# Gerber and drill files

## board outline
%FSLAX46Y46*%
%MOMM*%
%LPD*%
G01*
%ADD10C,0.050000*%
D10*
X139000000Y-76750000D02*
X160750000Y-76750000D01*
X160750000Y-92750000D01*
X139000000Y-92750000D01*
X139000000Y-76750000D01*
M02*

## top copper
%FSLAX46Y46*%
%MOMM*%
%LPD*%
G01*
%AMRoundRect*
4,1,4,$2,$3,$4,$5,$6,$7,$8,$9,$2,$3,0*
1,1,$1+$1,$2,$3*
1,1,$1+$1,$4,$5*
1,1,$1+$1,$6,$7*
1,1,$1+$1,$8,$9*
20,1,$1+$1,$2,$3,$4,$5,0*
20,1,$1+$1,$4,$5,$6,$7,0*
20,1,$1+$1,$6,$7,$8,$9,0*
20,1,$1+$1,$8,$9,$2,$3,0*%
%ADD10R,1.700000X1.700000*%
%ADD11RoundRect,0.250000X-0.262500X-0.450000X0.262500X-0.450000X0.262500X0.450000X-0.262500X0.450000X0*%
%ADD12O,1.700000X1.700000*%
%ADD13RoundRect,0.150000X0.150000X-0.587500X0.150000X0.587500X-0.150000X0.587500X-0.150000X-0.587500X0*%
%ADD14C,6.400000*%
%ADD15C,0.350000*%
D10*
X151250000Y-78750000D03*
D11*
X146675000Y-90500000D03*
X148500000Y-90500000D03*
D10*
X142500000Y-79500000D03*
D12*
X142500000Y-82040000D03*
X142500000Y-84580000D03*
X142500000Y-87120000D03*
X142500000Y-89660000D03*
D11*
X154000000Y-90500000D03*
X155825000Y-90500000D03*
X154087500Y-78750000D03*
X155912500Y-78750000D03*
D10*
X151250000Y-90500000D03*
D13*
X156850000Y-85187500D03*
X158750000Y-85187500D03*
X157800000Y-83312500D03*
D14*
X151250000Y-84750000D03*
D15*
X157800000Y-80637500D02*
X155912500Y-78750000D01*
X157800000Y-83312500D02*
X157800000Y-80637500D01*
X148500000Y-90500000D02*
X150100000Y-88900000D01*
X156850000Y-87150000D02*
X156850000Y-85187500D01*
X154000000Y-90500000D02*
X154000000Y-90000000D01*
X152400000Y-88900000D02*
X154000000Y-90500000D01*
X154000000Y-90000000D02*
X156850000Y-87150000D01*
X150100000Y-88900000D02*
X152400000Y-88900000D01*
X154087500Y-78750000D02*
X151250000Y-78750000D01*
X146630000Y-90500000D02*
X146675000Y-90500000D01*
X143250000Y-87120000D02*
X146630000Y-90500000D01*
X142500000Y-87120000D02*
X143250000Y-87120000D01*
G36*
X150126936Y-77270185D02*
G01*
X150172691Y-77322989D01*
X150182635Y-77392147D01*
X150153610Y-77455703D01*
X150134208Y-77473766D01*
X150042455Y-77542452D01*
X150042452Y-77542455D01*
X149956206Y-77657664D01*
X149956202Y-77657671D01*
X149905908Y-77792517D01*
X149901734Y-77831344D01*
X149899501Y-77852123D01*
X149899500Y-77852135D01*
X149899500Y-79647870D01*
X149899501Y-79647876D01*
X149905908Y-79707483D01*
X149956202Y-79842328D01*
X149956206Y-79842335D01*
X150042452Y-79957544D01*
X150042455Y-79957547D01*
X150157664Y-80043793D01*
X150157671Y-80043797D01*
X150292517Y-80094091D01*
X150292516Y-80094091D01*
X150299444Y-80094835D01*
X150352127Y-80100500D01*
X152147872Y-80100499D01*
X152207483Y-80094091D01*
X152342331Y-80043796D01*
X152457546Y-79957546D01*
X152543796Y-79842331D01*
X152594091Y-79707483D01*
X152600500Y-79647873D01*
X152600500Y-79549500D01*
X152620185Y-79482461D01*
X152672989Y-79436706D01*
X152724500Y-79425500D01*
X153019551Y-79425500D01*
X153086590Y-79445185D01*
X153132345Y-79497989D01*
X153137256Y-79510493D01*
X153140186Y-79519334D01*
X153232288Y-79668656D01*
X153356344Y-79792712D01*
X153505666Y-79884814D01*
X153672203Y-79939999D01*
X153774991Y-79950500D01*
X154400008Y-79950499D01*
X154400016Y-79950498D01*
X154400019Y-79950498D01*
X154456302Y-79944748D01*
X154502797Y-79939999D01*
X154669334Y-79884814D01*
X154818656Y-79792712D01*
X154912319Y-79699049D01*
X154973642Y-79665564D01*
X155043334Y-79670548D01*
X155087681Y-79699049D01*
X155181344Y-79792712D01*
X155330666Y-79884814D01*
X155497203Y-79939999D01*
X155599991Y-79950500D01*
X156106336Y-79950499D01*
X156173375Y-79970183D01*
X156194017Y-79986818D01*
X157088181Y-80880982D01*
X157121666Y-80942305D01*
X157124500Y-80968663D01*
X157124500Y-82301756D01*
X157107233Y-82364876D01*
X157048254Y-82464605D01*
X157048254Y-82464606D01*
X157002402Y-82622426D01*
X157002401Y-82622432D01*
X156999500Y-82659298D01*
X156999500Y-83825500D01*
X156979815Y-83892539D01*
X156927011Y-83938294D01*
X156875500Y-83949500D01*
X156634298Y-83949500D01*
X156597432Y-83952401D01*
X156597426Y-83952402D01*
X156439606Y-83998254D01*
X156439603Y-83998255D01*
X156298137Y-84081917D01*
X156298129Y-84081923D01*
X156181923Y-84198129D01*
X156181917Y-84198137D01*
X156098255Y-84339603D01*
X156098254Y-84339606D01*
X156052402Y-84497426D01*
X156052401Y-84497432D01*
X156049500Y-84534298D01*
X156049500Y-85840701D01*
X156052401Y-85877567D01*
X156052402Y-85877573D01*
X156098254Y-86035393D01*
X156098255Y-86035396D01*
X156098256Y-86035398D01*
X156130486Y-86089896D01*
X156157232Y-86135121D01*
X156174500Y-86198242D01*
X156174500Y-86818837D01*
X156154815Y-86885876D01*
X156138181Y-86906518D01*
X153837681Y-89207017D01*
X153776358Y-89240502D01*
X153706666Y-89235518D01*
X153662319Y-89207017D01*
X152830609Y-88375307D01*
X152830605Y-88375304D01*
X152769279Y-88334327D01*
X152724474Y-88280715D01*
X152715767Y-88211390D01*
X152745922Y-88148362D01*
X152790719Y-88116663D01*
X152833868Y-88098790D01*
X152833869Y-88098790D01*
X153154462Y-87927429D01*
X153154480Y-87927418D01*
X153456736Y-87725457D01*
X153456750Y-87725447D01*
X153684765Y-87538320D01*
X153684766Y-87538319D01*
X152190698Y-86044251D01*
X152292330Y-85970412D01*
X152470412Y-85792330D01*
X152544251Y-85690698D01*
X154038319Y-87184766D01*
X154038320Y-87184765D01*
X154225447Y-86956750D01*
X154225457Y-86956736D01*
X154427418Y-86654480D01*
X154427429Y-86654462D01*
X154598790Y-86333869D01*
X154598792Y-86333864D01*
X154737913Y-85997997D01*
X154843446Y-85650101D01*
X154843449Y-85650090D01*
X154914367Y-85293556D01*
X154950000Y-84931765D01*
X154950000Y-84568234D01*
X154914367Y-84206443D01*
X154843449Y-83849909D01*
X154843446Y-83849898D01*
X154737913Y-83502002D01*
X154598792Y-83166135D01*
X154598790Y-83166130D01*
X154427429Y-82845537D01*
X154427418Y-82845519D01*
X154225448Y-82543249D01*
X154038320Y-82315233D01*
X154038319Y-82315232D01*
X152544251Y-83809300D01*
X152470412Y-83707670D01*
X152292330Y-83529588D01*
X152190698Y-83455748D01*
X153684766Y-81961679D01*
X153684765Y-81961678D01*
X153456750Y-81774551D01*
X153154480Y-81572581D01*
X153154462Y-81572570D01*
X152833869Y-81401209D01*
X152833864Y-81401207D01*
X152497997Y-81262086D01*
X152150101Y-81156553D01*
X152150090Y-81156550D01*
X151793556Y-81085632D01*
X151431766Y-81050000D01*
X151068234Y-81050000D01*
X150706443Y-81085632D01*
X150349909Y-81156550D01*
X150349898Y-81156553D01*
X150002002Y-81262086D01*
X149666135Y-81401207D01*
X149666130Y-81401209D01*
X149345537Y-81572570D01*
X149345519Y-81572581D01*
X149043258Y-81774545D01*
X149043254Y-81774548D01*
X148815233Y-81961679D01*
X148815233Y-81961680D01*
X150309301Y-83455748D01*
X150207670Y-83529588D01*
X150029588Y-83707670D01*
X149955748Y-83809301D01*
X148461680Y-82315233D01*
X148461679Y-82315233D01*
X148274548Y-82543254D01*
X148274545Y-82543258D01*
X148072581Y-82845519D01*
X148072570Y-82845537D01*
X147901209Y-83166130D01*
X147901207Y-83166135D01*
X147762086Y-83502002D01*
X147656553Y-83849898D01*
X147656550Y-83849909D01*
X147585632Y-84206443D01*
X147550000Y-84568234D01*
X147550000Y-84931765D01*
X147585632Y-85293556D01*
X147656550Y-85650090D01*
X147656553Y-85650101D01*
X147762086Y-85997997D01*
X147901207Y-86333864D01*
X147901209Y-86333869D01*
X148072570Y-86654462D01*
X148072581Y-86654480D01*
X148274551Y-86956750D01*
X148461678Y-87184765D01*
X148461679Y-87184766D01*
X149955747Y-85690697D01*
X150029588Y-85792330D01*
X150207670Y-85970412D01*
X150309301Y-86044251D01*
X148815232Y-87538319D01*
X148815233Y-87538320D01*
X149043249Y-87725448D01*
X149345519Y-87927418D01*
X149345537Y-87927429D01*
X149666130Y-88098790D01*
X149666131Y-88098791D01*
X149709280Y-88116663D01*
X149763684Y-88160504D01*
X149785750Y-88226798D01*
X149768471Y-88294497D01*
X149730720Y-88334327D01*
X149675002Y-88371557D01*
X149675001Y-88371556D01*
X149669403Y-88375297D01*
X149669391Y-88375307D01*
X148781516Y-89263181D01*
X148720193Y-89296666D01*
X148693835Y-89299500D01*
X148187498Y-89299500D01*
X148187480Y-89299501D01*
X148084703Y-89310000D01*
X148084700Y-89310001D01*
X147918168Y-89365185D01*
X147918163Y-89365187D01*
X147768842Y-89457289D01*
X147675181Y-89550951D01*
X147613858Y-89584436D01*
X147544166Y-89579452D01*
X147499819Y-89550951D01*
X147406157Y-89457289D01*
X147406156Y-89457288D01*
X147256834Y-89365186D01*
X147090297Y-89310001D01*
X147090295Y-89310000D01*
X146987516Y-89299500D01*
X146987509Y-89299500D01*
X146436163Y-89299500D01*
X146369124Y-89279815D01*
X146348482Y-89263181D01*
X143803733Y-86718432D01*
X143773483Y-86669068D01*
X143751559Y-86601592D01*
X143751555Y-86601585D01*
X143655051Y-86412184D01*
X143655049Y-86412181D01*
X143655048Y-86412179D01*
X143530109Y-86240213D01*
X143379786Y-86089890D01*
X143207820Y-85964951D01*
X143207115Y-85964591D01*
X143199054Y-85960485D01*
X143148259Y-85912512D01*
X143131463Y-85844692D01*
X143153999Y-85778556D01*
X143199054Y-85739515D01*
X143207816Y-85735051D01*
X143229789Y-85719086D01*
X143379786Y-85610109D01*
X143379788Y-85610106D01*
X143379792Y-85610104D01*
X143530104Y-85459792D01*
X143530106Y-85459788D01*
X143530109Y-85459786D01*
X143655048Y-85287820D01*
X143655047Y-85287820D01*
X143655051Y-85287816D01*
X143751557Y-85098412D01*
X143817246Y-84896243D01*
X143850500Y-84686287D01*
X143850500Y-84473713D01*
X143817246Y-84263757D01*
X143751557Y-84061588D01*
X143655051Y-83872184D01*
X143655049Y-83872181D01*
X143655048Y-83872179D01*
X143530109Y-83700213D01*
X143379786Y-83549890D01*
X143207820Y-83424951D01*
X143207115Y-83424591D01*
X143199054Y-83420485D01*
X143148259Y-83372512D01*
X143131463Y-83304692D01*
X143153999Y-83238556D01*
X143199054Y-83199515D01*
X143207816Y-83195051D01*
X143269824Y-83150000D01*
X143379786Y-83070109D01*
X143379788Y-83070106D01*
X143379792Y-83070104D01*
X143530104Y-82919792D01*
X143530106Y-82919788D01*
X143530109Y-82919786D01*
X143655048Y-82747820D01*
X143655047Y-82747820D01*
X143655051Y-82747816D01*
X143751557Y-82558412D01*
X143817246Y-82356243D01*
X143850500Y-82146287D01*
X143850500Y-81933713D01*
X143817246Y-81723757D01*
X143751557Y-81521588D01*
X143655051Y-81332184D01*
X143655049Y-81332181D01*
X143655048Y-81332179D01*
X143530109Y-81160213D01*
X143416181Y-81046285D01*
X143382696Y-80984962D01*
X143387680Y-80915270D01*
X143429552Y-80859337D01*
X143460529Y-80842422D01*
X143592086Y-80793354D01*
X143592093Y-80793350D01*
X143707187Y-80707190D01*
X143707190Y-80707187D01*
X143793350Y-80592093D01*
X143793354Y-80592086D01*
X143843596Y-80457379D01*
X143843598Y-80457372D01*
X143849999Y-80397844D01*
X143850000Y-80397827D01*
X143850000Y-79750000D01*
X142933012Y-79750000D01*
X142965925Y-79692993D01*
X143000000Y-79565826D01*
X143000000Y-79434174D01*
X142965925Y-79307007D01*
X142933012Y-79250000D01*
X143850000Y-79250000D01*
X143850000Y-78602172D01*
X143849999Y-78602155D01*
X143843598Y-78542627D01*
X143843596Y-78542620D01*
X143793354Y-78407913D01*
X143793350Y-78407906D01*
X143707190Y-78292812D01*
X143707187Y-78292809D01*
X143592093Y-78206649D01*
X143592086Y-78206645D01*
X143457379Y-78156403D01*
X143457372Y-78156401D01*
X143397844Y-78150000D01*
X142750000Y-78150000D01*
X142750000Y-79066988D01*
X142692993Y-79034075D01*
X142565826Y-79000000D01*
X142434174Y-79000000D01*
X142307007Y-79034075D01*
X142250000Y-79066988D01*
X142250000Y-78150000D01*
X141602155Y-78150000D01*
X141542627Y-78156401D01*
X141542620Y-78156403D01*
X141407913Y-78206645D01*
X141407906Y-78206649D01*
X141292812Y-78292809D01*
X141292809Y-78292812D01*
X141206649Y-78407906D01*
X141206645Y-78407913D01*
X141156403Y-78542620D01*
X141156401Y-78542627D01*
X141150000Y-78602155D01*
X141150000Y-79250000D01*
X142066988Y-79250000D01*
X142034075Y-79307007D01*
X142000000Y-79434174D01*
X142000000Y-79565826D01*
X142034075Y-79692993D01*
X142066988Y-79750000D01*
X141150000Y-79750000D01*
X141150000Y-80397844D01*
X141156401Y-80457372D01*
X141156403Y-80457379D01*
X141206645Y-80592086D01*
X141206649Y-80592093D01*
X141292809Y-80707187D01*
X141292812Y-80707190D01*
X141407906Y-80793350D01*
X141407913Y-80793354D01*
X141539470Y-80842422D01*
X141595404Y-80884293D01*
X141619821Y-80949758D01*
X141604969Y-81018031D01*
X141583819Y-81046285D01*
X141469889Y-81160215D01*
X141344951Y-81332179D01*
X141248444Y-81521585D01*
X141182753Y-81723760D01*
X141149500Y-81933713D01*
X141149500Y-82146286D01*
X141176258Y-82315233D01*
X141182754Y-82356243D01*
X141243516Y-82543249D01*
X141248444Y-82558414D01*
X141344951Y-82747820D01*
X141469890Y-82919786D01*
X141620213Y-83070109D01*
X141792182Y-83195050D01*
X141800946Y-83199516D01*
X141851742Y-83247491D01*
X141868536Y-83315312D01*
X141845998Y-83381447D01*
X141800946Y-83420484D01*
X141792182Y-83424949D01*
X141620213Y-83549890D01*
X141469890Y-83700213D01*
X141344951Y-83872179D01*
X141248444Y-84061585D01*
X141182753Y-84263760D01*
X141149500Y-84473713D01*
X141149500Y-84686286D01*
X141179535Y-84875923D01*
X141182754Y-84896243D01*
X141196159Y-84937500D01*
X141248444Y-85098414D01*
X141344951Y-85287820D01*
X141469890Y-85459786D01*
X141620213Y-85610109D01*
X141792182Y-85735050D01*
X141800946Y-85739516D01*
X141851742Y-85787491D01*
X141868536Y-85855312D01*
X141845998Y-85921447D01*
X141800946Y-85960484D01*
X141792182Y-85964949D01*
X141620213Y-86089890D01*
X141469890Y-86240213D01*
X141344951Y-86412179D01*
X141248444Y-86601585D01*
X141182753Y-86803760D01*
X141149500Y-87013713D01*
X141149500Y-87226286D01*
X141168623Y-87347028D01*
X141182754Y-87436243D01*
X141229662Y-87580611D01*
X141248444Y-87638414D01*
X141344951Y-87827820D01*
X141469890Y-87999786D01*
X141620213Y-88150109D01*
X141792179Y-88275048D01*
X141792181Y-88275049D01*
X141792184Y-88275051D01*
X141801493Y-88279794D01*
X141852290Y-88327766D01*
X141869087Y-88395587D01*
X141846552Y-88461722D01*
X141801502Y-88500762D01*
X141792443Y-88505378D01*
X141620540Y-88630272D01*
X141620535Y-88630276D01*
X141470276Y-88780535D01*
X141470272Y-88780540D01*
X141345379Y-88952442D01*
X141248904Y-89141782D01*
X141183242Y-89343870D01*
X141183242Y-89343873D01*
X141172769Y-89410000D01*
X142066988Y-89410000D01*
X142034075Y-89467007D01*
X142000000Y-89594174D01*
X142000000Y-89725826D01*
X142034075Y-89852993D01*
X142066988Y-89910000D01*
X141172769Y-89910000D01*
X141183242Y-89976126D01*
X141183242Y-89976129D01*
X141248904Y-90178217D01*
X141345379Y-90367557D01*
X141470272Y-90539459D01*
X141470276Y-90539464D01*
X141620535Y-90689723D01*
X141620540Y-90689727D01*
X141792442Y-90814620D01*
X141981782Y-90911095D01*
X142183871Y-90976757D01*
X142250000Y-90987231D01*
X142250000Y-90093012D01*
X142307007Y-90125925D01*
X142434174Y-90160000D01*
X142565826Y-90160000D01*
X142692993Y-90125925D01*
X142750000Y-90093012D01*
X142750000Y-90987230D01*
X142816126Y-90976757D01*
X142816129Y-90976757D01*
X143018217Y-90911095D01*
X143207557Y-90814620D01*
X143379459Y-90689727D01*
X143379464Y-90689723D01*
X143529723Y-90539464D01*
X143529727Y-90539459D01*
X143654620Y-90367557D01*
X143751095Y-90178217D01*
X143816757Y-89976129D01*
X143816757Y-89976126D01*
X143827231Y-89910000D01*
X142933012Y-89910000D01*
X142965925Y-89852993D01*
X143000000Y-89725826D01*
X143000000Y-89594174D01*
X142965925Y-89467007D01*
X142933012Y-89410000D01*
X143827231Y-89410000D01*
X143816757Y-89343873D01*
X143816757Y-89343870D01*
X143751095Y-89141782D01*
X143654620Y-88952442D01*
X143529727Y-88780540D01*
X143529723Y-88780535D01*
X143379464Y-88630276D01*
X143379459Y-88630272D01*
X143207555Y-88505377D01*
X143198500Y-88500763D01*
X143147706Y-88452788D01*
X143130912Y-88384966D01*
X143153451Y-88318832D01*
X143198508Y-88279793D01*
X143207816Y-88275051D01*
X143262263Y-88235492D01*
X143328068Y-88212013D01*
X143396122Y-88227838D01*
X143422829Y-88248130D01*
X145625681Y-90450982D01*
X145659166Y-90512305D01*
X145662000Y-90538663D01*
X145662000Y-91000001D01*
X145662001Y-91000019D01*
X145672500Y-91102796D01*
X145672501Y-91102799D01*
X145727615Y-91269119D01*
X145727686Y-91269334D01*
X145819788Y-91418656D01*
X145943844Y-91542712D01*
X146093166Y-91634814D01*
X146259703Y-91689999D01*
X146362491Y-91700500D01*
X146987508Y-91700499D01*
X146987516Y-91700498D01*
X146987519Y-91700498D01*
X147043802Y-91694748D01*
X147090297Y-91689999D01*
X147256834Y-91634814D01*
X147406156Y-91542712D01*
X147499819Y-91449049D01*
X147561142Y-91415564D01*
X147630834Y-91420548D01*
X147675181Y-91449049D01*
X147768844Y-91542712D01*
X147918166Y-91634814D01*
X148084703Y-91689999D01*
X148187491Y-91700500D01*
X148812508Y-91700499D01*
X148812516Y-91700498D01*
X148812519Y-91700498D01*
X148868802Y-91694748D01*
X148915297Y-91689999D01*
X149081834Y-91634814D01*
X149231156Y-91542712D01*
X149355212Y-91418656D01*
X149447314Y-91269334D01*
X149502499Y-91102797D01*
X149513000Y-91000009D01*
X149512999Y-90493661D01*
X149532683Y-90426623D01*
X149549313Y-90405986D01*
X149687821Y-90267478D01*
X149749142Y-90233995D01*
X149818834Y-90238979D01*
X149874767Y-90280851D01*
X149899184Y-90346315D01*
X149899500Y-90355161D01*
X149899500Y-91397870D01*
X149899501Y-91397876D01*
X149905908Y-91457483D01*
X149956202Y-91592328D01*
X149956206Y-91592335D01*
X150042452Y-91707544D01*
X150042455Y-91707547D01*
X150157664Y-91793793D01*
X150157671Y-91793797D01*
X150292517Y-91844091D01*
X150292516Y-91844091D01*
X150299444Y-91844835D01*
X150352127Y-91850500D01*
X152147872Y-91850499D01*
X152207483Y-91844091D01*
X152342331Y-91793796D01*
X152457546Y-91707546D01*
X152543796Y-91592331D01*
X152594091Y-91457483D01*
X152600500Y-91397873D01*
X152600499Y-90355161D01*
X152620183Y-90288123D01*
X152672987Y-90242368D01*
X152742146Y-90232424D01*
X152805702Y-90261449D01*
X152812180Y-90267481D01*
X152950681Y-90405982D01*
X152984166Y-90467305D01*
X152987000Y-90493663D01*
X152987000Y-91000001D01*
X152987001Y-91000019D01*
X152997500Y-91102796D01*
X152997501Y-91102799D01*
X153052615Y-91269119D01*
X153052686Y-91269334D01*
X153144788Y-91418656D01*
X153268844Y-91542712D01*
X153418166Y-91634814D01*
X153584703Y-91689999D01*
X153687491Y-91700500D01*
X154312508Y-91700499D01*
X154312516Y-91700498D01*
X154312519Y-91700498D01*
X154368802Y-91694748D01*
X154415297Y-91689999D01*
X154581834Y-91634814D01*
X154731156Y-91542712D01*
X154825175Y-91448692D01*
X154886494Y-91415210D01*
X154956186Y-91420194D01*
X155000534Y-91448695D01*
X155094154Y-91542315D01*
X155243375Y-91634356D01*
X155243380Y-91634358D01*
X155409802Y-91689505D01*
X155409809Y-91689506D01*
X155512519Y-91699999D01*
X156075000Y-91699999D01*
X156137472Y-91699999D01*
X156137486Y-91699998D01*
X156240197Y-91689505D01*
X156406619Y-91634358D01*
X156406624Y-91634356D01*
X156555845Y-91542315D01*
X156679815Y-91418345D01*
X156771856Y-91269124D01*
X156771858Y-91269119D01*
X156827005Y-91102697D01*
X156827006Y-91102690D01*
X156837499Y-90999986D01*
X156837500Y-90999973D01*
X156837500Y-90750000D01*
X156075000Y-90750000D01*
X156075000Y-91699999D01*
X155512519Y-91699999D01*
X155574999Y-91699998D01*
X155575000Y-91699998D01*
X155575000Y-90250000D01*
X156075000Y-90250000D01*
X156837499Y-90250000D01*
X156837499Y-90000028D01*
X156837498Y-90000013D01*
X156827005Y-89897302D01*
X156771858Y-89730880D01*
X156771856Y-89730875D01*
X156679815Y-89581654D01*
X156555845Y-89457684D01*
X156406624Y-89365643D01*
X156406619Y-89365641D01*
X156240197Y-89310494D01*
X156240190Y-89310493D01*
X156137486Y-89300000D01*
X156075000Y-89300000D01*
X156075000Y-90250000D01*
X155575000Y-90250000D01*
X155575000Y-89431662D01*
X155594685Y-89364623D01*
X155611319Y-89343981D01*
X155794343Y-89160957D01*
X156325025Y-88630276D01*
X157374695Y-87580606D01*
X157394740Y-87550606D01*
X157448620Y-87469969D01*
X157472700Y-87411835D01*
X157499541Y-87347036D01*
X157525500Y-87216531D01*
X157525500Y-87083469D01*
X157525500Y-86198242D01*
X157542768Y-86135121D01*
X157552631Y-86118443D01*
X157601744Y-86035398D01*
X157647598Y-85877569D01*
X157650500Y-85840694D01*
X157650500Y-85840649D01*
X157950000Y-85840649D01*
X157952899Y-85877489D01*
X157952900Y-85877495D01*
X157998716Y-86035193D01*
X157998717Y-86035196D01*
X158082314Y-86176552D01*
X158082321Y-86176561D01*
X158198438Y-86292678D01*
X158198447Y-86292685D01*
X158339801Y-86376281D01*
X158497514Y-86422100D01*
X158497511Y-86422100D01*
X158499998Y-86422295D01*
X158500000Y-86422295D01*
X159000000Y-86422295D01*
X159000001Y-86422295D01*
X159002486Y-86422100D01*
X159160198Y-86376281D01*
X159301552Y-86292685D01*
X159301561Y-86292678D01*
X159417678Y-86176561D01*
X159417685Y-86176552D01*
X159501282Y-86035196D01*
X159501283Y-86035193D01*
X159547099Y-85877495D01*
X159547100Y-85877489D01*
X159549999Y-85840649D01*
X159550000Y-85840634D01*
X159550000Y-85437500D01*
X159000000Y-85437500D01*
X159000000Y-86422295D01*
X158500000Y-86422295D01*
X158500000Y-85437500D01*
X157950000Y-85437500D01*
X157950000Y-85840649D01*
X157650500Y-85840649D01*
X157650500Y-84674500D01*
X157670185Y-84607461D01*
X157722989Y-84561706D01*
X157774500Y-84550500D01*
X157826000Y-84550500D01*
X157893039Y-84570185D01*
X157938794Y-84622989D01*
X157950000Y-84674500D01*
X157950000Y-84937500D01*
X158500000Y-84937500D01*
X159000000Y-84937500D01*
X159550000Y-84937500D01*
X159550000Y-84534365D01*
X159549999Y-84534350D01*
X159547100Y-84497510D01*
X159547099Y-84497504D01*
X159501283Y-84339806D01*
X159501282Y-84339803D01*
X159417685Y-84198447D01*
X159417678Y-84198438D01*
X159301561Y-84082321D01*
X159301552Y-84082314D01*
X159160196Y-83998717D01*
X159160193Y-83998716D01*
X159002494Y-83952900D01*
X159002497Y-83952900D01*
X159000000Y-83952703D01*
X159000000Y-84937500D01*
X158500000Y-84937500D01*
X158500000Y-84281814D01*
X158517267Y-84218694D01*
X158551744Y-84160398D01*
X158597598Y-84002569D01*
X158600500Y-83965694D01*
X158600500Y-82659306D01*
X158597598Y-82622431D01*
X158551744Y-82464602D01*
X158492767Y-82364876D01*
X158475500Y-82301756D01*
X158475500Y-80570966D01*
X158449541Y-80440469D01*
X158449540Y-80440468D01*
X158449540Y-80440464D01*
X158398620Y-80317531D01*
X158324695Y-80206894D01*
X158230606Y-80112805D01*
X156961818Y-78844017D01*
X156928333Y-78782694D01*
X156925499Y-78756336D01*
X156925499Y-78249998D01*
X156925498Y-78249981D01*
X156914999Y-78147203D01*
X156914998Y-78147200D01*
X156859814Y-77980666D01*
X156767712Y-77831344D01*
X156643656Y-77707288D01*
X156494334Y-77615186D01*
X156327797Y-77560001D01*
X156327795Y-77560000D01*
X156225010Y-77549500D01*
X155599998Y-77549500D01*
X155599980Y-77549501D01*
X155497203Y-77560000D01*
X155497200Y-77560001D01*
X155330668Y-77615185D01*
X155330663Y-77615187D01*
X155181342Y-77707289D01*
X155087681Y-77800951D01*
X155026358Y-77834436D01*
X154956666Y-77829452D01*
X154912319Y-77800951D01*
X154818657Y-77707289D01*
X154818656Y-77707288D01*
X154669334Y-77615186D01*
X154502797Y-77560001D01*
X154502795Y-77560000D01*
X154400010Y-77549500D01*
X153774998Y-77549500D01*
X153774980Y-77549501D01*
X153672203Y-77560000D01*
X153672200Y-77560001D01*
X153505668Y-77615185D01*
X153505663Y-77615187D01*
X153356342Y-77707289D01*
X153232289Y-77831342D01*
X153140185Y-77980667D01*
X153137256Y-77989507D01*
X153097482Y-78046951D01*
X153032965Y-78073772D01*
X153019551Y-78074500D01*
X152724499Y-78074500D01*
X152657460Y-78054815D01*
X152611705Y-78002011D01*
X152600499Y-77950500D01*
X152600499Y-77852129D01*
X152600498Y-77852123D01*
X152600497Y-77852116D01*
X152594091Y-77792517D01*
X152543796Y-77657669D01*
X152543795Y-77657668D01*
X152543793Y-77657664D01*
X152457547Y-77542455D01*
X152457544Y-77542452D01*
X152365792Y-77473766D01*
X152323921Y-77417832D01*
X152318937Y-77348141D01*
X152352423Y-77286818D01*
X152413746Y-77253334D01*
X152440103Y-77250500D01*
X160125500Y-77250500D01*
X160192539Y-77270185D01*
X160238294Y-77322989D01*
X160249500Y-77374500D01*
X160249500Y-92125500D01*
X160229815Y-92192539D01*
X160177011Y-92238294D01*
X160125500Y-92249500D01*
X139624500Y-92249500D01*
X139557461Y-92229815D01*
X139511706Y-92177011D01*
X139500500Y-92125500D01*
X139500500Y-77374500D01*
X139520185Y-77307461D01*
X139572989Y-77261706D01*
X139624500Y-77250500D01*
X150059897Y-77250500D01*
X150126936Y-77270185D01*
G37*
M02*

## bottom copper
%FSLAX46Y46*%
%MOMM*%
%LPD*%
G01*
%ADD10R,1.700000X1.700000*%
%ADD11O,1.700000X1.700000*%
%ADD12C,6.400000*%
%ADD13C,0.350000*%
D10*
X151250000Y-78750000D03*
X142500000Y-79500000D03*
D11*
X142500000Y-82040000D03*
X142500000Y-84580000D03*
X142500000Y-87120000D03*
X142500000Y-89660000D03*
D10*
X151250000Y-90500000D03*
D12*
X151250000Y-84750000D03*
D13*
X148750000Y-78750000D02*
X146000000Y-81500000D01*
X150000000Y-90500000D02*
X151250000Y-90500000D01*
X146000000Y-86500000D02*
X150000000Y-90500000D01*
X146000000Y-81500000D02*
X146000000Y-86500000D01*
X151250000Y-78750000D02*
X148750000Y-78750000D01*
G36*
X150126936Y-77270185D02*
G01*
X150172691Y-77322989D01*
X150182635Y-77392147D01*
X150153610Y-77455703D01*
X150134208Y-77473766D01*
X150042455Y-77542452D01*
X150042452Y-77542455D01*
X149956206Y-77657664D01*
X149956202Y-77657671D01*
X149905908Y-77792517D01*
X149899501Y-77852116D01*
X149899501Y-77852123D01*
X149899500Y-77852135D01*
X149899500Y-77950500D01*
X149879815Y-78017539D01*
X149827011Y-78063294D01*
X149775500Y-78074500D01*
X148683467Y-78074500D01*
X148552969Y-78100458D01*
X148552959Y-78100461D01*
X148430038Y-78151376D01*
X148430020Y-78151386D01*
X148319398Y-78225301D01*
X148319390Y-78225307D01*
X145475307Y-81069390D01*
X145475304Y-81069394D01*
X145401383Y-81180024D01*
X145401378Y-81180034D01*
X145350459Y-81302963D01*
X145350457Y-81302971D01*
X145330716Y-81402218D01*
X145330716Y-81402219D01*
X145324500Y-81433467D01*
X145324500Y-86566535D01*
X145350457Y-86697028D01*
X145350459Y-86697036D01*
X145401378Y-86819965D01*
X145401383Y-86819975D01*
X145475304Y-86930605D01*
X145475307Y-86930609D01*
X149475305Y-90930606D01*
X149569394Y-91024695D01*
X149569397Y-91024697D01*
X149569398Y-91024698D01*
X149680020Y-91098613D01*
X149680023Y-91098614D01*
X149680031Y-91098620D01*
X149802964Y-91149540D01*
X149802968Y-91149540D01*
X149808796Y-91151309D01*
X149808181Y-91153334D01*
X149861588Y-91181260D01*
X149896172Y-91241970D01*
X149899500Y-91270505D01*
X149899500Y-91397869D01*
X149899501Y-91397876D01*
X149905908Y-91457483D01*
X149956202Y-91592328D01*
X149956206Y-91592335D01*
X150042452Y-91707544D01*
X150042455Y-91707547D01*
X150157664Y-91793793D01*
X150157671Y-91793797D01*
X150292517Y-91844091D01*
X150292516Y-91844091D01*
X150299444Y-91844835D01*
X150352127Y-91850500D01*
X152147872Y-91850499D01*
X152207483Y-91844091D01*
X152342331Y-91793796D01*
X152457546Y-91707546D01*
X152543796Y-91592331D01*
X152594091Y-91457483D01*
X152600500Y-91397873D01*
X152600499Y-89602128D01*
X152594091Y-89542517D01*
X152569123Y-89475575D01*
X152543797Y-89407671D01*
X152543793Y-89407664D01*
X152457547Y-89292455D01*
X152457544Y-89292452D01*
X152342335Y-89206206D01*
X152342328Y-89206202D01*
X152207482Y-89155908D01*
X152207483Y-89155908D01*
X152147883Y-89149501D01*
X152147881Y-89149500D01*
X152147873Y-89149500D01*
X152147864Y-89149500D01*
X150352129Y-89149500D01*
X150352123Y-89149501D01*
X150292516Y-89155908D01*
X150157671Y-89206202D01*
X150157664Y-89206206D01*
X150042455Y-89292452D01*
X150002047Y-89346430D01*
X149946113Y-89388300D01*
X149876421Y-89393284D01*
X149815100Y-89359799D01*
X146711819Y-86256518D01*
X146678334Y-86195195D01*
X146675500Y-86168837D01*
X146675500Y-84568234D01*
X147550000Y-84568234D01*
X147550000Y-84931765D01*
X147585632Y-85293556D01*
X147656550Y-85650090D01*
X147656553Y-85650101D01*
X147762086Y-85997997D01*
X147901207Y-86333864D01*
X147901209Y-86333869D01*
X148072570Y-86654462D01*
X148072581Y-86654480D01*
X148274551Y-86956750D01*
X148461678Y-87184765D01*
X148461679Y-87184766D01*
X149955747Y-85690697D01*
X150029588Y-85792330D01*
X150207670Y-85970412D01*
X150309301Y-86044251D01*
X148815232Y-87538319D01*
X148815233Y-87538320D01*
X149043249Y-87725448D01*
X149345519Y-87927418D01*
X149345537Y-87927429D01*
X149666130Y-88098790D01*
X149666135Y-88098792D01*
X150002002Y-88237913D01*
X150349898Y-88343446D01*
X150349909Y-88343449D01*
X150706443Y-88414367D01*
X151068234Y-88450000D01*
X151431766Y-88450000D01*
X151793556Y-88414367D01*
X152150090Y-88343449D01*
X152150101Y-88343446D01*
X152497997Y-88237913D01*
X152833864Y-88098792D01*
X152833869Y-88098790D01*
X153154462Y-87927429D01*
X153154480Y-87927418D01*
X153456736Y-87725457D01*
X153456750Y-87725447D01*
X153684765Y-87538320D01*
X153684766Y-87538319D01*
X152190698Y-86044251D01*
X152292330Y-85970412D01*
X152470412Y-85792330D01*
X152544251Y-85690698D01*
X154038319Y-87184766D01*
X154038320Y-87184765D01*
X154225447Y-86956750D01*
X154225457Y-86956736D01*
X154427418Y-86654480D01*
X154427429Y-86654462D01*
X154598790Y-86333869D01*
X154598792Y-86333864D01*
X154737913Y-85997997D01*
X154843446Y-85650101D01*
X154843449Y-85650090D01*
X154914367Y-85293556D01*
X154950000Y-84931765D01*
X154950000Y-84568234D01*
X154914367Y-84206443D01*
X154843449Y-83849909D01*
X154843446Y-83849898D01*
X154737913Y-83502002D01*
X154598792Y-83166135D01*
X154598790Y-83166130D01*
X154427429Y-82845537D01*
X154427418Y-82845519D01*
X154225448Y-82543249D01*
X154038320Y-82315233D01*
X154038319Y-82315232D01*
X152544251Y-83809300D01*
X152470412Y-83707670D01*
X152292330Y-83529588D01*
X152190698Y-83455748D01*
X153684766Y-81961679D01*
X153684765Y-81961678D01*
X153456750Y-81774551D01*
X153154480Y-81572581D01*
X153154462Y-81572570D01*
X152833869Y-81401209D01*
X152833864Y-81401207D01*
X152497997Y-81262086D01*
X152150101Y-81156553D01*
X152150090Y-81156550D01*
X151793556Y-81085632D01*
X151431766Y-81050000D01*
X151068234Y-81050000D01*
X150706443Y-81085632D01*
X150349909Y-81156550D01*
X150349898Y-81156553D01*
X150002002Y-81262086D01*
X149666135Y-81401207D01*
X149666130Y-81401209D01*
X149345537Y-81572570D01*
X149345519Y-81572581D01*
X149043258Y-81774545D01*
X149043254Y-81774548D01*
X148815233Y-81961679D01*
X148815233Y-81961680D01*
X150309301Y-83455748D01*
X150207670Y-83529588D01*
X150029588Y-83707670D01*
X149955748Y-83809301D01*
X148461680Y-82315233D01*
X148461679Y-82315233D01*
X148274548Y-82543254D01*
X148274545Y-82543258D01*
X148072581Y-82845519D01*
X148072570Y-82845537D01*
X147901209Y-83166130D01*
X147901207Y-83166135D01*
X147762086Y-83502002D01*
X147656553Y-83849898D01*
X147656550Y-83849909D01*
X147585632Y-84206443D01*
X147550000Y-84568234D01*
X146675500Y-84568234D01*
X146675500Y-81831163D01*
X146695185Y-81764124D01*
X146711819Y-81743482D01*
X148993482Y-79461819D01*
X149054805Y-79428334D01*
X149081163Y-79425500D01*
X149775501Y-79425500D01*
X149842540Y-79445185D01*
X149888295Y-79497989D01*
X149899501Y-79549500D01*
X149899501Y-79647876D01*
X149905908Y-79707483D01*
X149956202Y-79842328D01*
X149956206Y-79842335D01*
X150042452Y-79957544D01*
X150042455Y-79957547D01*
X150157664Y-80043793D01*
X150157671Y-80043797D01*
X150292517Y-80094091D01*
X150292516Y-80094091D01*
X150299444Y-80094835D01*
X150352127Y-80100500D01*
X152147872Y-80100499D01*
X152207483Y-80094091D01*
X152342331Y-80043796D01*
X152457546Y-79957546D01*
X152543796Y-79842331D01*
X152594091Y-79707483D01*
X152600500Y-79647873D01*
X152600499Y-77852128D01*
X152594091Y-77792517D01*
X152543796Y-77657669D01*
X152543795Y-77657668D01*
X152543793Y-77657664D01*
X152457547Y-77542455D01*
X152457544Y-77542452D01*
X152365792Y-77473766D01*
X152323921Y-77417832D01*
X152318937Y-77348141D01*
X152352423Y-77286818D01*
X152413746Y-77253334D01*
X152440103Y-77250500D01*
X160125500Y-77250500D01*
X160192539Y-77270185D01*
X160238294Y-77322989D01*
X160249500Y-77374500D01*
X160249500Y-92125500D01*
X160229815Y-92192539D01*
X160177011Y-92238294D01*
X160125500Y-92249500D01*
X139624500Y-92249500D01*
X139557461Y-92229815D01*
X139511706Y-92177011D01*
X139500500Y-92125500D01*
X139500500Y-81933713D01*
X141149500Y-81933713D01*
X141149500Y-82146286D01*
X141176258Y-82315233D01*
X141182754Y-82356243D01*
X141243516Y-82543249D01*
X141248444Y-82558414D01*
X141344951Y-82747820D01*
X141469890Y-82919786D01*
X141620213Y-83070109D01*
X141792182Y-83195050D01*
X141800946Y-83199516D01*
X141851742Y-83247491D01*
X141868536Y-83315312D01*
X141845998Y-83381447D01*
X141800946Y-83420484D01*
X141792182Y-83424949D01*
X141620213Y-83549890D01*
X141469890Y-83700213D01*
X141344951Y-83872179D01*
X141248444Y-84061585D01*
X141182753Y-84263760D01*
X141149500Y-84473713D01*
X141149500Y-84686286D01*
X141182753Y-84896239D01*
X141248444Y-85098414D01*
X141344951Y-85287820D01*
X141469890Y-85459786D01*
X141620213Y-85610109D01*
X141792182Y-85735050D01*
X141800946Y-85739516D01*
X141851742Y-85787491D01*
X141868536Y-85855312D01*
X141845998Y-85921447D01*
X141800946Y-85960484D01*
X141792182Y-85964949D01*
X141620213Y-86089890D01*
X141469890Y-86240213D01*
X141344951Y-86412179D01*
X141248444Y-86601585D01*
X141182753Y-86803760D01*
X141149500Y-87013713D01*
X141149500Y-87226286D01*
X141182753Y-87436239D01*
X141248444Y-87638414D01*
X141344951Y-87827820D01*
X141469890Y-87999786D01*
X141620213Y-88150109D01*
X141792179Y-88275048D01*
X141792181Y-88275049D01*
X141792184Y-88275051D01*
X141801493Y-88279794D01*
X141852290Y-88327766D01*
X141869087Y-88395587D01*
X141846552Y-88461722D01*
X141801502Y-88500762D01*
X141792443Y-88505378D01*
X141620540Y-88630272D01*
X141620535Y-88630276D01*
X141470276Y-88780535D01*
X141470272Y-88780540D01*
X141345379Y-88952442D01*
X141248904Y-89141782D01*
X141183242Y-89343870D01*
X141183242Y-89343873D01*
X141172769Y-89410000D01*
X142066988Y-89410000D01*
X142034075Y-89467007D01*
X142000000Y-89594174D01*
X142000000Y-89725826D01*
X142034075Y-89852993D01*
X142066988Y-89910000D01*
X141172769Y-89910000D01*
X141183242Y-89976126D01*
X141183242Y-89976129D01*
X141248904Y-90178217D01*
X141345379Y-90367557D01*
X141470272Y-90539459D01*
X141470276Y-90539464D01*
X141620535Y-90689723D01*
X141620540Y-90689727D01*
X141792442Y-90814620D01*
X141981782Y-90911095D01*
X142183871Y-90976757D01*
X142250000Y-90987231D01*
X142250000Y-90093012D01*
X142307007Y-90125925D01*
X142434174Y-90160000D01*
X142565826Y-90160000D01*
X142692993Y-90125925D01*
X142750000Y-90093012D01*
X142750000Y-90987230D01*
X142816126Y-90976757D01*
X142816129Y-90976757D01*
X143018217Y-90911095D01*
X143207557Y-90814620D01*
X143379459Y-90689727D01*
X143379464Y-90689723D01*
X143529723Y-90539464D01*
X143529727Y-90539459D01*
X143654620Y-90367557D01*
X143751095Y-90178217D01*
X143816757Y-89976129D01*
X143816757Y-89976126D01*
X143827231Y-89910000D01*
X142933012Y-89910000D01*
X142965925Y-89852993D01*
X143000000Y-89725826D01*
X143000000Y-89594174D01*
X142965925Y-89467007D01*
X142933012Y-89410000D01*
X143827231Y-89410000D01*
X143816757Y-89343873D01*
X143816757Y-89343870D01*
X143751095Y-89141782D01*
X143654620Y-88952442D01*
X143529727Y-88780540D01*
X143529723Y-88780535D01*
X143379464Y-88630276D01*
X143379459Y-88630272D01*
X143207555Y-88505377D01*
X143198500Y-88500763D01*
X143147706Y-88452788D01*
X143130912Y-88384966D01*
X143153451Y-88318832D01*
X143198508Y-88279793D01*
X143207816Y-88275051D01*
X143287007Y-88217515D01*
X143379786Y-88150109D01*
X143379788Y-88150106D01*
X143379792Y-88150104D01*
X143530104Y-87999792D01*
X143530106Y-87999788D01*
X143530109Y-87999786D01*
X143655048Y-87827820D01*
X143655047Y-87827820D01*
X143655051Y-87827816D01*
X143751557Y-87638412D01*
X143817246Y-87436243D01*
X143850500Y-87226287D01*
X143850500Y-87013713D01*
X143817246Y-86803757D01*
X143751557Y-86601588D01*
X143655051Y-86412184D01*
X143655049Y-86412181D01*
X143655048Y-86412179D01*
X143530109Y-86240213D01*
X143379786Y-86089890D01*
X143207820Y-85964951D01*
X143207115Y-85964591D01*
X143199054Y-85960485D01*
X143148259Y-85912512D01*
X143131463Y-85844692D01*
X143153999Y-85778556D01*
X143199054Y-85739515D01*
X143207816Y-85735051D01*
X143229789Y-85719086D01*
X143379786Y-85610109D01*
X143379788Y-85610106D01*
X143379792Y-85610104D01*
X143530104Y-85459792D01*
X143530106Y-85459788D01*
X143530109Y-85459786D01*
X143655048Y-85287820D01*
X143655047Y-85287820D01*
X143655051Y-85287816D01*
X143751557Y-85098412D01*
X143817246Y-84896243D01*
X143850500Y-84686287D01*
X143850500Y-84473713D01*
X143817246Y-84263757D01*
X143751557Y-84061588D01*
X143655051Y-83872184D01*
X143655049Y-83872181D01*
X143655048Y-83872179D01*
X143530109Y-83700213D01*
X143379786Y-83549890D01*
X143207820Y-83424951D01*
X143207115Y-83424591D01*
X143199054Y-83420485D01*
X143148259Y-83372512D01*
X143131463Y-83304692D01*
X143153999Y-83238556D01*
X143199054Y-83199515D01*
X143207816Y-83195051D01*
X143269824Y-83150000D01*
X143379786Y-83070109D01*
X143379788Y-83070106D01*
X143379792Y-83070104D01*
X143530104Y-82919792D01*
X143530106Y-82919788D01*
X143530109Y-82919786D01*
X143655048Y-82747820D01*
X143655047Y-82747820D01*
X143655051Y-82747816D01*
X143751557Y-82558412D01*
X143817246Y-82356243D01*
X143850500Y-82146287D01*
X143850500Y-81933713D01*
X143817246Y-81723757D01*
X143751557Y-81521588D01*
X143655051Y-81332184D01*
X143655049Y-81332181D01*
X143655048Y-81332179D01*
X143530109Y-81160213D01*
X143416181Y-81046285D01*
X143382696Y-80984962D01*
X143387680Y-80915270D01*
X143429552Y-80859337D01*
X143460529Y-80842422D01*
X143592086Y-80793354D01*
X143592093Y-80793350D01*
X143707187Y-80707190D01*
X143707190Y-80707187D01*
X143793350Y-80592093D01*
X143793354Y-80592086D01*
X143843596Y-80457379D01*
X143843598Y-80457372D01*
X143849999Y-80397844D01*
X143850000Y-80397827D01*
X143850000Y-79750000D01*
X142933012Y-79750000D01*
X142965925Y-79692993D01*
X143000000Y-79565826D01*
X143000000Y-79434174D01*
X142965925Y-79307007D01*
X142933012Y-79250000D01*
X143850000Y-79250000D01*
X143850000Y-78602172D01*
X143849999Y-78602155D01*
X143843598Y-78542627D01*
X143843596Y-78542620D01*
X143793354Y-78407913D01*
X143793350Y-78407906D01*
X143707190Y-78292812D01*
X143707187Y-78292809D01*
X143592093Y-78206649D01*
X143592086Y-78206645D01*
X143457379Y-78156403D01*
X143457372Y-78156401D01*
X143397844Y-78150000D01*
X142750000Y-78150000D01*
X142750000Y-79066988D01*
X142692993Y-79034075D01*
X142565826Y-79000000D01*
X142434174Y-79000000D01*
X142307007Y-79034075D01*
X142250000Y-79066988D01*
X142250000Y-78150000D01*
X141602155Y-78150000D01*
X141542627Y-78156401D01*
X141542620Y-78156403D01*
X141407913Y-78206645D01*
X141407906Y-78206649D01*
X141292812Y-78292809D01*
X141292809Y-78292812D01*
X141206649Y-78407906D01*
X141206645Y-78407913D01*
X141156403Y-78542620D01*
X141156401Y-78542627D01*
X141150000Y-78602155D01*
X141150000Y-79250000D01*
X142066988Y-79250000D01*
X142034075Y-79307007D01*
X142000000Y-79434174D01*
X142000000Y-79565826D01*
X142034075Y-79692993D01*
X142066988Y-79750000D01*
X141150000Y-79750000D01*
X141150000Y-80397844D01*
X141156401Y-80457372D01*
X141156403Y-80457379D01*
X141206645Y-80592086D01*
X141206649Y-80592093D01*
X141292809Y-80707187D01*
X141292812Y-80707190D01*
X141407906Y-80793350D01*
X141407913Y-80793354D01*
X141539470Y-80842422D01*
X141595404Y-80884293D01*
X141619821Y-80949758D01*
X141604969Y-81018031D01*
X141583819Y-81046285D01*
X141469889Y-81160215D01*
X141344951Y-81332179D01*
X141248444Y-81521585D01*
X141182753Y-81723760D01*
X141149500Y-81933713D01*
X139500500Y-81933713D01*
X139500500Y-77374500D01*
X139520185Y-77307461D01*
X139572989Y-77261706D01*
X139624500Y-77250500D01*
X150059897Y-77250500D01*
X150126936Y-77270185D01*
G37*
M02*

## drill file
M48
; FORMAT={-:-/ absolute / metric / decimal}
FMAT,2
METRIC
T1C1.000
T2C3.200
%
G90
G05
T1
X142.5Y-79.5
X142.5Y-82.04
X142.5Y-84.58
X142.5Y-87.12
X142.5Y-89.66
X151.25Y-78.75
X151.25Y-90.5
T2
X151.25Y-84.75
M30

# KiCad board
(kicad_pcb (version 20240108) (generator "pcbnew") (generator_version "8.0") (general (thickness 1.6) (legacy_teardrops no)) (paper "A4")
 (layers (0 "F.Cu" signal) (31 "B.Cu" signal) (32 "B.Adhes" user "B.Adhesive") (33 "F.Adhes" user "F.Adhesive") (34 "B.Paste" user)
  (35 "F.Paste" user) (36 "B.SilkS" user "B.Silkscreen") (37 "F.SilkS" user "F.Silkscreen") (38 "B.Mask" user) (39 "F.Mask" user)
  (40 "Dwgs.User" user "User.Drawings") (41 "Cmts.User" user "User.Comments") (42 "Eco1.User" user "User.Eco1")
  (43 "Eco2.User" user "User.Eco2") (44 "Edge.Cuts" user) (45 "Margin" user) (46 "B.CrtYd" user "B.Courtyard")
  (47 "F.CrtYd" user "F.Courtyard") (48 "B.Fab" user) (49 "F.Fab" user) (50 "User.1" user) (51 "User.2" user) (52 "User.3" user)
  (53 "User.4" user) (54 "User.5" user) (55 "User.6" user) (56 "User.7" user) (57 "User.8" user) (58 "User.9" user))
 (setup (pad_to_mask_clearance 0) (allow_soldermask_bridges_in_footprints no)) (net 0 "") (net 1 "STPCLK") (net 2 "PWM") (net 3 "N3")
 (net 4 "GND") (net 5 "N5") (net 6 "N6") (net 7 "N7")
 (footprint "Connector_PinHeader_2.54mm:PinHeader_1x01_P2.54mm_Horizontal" (layer "F.Cu") (at 151.25 78.75 90)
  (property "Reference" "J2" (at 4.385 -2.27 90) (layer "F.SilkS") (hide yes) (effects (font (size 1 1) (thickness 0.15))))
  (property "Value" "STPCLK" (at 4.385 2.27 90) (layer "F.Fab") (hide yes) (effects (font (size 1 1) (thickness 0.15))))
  (pad "1" thru_hole rect (at 0 0 90) (size 1.7 1.7) (drill 1) (layers "*.Cu" "*.Mask") (remove_unused_layers no) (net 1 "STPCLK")))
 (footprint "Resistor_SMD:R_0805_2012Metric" (layer "F.Cu") (at 147.5875 90.5)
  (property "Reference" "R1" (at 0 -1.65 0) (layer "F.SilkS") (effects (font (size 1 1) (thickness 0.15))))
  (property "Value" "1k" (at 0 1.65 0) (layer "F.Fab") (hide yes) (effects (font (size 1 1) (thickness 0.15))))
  (pad "1" smd roundrect (at -0.9125 0) (size 1.025 1.4) (layers "F.Cu" "F.Paste" "F.Mask") (roundrect_rratio 0.243902) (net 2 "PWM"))
  (pad "2" smd roundrect (at 0.9125 0) (size 1.025 1.4) (layers "F.Cu" "F.Paste" "F.Mask") (roundrect_rratio 0.243902) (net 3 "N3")))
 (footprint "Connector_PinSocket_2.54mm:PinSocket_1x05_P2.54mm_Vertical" (layer "F.Cu") (at 142.5 79.5)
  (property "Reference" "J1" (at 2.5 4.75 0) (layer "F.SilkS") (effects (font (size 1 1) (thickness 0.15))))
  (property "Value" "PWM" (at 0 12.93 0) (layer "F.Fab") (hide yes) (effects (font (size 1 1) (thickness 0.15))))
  (pad "1" thru_hole rect (at 0 0) (size 1.7 1.7) (drill 1) (layers "*.Cu" "*.Mask") (remove_unused_layers no) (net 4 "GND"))
  (pad "2" thru_hole oval (at 0 2.54) (size 1.7 1.7) (drill 1) (layers "*.Cu" "*.Mask") (remove_unused_layers no) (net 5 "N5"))
  (pad "3" thru_hole oval (at 0 5.08) (size 1.7 1.7) (drill 1) (layers "*.Cu" "*.Mask") (remove_unused_layers no) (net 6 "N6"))
  (pad "4" thru_hole oval (at 0 7.62) (size 1.7 1.7) (drill 1) (layers "*.Cu" "*.Mask") (remove_unused_layers no) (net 2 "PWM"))
  (pad "5" thru_hole oval (at 0 10.16) (size 1.7 1.7) (drill 1) (layers "*.Cu" "*.Mask") (remove_unused_layers no) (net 4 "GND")))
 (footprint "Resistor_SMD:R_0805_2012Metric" (layer "F.Cu") (at 154.9125 90.5)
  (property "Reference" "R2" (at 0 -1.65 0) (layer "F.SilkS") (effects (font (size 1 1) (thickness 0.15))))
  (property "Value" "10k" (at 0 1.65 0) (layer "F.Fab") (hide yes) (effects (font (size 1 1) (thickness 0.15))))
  (pad "1" smd roundrect (at -0.9125 0) (size 1.025 1.4) (layers "F.Cu" "F.Paste" "F.Mask") (roundrect_rratio 0.243902) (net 3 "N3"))
  (pad "2" smd roundrect (at 0.9125 0) (size 1.025 1.4) (layers "F.Cu" "F.Paste" "F.Mask") (roundrect_rratio 0.243902) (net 4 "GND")))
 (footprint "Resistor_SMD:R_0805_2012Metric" (layer "F.Cu") (at 155 78.75)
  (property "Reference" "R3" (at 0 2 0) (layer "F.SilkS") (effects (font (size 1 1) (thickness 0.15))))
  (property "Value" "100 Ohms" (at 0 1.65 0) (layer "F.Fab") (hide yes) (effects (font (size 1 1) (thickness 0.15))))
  (pad "1" smd roundrect (at -0.9125 0) (size 1.025 1.4) (layers "F.Cu" "F.Paste" "F.Mask") (roundrect_rratio 0.243902) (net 1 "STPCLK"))
  (pad "2" smd roundrect (at 0.9125 0) (size 1.025 1.4) (layers "F.Cu" "F.Paste" "F.Mask") (roundrect_rratio 0.243902) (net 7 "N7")))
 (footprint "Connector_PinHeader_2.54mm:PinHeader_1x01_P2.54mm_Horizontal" (layer "F.Cu") (at 151.25 90.5 -90)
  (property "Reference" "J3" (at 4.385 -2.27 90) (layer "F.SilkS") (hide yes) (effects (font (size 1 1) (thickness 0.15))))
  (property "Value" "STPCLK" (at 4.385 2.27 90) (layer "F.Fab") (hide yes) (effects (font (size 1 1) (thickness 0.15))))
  (pad "1" thru_hole rect (at 0 0 270) (size 1.7 1.7) (drill 1) (layers "*.Cu" "*.Mask") (remove_unused_layers no) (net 1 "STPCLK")))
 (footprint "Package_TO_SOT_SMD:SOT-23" (layer "F.Cu") (at 157.8 84.25 90)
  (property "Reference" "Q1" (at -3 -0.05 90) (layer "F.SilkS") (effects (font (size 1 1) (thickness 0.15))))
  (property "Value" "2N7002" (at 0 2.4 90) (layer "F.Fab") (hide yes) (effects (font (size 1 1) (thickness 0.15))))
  (pad "1" smd roundrect (at -0.9375 -0.95 90) (size 1.475 0.6) (layers "F.Cu" "F.Paste" "F.Mask") (roundrect_rratio 0.25) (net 3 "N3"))
  (pad "2" smd roundrect (at -0.9375 0.95 90) (size 1.475 0.6) (layers "F.Cu" "F.Paste" "F.Mask") (roundrect_rratio 0.25) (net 4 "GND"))
  (pad "3" smd roundrect (at 0.9375 0 90) (size 1.475 0.6) (layers "F.Cu" "F.Paste" "F.Mask") (roundrect_rratio 0.25) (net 7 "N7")))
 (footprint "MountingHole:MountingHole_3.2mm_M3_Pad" (layer "F.Cu") (at 151.25 84.75)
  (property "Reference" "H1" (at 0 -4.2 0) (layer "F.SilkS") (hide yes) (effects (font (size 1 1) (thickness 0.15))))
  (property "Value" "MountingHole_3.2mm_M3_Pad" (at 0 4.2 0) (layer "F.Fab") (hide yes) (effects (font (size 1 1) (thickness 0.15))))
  (pad "1" thru_hole circle (at 0 0) (size 6.4 6.4) (drill 3.2) (layers "*.Cu" "*.Mask") (remove_unused_layers no) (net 4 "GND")))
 (gr_rect (start 139 76.75) (end 160.75 92.75) (stroke (width 0.05) (type default)) (fill none) (layer "Edge.Cuts"))
 (segment (start 157.8 80.6375) (end 155.9125 78.75) (width 0.35) (layer "F.Cu") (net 7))
 (segment (start 157.8 83.3125) (end 157.8 80.6375) (width 0.35) (layer "F.Cu") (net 7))
 (segment (start 148.5 90.5) (end 150.1 88.9) (width 0.35) (layer "F.Cu") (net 3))
 (segment (start 156.85 87.15) (end 156.85 85.1875) (width 0.35) (layer "F.Cu") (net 3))
 (segment (start 154 90.5) (end 154 90) (width 0.35) (layer "F.Cu") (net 3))
 (segment (start 152.4 88.9) (end 154 90.5) (width 0.35) (layer "F.Cu") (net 3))
 (segment (start 154 90) (end 156.85 87.15) (width 0.35) (layer "F.Cu") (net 3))
 (segment (start 150.1 88.9) (end 152.4 88.9) (width 0.35) (layer "F.Cu") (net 3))
 (segment (start 154.0875 78.75) (end 151.25 78.75) (width 0.35) (layer "F.Cu") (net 1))
 (segment (start 148.75 78.75) (end 146 81.5) (width 0.35) (layer "B.Cu") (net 1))
 (segment (start 150 90.5) (end 151.25 90.5) (width 0.35) (layer "B.Cu") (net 1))
 (segment (start 146 86.5) (end 150 90.5) (width 0.35) (layer "B.Cu") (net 1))
 (segment (start 146 81.5) (end 146 86.5) (width 0.35) (layer "B.Cu") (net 1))
 (segment (start 151.25 78.75) (end 148.75 78.75) (width 0.35) (layer "B.Cu") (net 1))
 (segment (start 146.63 90.5) (end 146.675 90.5) (width 0.35) (layer "F.Cu") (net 2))
 (segment (start 143.25 87.12) (end 146.63 90.5) (width 0.35) (layer "F.Cu") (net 2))
 (segment (start 142.5 87.12) (end 143.25 87.12) (width 0.35) (layer "F.Cu") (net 2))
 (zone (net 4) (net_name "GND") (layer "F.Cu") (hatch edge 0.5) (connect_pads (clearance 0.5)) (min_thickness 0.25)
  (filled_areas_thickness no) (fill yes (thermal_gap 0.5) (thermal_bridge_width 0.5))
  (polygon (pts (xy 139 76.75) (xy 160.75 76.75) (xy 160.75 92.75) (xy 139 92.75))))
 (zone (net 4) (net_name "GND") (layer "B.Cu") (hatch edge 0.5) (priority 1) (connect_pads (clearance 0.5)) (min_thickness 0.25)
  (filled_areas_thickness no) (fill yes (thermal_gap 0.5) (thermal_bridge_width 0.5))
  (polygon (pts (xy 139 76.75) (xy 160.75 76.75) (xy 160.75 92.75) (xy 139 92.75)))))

